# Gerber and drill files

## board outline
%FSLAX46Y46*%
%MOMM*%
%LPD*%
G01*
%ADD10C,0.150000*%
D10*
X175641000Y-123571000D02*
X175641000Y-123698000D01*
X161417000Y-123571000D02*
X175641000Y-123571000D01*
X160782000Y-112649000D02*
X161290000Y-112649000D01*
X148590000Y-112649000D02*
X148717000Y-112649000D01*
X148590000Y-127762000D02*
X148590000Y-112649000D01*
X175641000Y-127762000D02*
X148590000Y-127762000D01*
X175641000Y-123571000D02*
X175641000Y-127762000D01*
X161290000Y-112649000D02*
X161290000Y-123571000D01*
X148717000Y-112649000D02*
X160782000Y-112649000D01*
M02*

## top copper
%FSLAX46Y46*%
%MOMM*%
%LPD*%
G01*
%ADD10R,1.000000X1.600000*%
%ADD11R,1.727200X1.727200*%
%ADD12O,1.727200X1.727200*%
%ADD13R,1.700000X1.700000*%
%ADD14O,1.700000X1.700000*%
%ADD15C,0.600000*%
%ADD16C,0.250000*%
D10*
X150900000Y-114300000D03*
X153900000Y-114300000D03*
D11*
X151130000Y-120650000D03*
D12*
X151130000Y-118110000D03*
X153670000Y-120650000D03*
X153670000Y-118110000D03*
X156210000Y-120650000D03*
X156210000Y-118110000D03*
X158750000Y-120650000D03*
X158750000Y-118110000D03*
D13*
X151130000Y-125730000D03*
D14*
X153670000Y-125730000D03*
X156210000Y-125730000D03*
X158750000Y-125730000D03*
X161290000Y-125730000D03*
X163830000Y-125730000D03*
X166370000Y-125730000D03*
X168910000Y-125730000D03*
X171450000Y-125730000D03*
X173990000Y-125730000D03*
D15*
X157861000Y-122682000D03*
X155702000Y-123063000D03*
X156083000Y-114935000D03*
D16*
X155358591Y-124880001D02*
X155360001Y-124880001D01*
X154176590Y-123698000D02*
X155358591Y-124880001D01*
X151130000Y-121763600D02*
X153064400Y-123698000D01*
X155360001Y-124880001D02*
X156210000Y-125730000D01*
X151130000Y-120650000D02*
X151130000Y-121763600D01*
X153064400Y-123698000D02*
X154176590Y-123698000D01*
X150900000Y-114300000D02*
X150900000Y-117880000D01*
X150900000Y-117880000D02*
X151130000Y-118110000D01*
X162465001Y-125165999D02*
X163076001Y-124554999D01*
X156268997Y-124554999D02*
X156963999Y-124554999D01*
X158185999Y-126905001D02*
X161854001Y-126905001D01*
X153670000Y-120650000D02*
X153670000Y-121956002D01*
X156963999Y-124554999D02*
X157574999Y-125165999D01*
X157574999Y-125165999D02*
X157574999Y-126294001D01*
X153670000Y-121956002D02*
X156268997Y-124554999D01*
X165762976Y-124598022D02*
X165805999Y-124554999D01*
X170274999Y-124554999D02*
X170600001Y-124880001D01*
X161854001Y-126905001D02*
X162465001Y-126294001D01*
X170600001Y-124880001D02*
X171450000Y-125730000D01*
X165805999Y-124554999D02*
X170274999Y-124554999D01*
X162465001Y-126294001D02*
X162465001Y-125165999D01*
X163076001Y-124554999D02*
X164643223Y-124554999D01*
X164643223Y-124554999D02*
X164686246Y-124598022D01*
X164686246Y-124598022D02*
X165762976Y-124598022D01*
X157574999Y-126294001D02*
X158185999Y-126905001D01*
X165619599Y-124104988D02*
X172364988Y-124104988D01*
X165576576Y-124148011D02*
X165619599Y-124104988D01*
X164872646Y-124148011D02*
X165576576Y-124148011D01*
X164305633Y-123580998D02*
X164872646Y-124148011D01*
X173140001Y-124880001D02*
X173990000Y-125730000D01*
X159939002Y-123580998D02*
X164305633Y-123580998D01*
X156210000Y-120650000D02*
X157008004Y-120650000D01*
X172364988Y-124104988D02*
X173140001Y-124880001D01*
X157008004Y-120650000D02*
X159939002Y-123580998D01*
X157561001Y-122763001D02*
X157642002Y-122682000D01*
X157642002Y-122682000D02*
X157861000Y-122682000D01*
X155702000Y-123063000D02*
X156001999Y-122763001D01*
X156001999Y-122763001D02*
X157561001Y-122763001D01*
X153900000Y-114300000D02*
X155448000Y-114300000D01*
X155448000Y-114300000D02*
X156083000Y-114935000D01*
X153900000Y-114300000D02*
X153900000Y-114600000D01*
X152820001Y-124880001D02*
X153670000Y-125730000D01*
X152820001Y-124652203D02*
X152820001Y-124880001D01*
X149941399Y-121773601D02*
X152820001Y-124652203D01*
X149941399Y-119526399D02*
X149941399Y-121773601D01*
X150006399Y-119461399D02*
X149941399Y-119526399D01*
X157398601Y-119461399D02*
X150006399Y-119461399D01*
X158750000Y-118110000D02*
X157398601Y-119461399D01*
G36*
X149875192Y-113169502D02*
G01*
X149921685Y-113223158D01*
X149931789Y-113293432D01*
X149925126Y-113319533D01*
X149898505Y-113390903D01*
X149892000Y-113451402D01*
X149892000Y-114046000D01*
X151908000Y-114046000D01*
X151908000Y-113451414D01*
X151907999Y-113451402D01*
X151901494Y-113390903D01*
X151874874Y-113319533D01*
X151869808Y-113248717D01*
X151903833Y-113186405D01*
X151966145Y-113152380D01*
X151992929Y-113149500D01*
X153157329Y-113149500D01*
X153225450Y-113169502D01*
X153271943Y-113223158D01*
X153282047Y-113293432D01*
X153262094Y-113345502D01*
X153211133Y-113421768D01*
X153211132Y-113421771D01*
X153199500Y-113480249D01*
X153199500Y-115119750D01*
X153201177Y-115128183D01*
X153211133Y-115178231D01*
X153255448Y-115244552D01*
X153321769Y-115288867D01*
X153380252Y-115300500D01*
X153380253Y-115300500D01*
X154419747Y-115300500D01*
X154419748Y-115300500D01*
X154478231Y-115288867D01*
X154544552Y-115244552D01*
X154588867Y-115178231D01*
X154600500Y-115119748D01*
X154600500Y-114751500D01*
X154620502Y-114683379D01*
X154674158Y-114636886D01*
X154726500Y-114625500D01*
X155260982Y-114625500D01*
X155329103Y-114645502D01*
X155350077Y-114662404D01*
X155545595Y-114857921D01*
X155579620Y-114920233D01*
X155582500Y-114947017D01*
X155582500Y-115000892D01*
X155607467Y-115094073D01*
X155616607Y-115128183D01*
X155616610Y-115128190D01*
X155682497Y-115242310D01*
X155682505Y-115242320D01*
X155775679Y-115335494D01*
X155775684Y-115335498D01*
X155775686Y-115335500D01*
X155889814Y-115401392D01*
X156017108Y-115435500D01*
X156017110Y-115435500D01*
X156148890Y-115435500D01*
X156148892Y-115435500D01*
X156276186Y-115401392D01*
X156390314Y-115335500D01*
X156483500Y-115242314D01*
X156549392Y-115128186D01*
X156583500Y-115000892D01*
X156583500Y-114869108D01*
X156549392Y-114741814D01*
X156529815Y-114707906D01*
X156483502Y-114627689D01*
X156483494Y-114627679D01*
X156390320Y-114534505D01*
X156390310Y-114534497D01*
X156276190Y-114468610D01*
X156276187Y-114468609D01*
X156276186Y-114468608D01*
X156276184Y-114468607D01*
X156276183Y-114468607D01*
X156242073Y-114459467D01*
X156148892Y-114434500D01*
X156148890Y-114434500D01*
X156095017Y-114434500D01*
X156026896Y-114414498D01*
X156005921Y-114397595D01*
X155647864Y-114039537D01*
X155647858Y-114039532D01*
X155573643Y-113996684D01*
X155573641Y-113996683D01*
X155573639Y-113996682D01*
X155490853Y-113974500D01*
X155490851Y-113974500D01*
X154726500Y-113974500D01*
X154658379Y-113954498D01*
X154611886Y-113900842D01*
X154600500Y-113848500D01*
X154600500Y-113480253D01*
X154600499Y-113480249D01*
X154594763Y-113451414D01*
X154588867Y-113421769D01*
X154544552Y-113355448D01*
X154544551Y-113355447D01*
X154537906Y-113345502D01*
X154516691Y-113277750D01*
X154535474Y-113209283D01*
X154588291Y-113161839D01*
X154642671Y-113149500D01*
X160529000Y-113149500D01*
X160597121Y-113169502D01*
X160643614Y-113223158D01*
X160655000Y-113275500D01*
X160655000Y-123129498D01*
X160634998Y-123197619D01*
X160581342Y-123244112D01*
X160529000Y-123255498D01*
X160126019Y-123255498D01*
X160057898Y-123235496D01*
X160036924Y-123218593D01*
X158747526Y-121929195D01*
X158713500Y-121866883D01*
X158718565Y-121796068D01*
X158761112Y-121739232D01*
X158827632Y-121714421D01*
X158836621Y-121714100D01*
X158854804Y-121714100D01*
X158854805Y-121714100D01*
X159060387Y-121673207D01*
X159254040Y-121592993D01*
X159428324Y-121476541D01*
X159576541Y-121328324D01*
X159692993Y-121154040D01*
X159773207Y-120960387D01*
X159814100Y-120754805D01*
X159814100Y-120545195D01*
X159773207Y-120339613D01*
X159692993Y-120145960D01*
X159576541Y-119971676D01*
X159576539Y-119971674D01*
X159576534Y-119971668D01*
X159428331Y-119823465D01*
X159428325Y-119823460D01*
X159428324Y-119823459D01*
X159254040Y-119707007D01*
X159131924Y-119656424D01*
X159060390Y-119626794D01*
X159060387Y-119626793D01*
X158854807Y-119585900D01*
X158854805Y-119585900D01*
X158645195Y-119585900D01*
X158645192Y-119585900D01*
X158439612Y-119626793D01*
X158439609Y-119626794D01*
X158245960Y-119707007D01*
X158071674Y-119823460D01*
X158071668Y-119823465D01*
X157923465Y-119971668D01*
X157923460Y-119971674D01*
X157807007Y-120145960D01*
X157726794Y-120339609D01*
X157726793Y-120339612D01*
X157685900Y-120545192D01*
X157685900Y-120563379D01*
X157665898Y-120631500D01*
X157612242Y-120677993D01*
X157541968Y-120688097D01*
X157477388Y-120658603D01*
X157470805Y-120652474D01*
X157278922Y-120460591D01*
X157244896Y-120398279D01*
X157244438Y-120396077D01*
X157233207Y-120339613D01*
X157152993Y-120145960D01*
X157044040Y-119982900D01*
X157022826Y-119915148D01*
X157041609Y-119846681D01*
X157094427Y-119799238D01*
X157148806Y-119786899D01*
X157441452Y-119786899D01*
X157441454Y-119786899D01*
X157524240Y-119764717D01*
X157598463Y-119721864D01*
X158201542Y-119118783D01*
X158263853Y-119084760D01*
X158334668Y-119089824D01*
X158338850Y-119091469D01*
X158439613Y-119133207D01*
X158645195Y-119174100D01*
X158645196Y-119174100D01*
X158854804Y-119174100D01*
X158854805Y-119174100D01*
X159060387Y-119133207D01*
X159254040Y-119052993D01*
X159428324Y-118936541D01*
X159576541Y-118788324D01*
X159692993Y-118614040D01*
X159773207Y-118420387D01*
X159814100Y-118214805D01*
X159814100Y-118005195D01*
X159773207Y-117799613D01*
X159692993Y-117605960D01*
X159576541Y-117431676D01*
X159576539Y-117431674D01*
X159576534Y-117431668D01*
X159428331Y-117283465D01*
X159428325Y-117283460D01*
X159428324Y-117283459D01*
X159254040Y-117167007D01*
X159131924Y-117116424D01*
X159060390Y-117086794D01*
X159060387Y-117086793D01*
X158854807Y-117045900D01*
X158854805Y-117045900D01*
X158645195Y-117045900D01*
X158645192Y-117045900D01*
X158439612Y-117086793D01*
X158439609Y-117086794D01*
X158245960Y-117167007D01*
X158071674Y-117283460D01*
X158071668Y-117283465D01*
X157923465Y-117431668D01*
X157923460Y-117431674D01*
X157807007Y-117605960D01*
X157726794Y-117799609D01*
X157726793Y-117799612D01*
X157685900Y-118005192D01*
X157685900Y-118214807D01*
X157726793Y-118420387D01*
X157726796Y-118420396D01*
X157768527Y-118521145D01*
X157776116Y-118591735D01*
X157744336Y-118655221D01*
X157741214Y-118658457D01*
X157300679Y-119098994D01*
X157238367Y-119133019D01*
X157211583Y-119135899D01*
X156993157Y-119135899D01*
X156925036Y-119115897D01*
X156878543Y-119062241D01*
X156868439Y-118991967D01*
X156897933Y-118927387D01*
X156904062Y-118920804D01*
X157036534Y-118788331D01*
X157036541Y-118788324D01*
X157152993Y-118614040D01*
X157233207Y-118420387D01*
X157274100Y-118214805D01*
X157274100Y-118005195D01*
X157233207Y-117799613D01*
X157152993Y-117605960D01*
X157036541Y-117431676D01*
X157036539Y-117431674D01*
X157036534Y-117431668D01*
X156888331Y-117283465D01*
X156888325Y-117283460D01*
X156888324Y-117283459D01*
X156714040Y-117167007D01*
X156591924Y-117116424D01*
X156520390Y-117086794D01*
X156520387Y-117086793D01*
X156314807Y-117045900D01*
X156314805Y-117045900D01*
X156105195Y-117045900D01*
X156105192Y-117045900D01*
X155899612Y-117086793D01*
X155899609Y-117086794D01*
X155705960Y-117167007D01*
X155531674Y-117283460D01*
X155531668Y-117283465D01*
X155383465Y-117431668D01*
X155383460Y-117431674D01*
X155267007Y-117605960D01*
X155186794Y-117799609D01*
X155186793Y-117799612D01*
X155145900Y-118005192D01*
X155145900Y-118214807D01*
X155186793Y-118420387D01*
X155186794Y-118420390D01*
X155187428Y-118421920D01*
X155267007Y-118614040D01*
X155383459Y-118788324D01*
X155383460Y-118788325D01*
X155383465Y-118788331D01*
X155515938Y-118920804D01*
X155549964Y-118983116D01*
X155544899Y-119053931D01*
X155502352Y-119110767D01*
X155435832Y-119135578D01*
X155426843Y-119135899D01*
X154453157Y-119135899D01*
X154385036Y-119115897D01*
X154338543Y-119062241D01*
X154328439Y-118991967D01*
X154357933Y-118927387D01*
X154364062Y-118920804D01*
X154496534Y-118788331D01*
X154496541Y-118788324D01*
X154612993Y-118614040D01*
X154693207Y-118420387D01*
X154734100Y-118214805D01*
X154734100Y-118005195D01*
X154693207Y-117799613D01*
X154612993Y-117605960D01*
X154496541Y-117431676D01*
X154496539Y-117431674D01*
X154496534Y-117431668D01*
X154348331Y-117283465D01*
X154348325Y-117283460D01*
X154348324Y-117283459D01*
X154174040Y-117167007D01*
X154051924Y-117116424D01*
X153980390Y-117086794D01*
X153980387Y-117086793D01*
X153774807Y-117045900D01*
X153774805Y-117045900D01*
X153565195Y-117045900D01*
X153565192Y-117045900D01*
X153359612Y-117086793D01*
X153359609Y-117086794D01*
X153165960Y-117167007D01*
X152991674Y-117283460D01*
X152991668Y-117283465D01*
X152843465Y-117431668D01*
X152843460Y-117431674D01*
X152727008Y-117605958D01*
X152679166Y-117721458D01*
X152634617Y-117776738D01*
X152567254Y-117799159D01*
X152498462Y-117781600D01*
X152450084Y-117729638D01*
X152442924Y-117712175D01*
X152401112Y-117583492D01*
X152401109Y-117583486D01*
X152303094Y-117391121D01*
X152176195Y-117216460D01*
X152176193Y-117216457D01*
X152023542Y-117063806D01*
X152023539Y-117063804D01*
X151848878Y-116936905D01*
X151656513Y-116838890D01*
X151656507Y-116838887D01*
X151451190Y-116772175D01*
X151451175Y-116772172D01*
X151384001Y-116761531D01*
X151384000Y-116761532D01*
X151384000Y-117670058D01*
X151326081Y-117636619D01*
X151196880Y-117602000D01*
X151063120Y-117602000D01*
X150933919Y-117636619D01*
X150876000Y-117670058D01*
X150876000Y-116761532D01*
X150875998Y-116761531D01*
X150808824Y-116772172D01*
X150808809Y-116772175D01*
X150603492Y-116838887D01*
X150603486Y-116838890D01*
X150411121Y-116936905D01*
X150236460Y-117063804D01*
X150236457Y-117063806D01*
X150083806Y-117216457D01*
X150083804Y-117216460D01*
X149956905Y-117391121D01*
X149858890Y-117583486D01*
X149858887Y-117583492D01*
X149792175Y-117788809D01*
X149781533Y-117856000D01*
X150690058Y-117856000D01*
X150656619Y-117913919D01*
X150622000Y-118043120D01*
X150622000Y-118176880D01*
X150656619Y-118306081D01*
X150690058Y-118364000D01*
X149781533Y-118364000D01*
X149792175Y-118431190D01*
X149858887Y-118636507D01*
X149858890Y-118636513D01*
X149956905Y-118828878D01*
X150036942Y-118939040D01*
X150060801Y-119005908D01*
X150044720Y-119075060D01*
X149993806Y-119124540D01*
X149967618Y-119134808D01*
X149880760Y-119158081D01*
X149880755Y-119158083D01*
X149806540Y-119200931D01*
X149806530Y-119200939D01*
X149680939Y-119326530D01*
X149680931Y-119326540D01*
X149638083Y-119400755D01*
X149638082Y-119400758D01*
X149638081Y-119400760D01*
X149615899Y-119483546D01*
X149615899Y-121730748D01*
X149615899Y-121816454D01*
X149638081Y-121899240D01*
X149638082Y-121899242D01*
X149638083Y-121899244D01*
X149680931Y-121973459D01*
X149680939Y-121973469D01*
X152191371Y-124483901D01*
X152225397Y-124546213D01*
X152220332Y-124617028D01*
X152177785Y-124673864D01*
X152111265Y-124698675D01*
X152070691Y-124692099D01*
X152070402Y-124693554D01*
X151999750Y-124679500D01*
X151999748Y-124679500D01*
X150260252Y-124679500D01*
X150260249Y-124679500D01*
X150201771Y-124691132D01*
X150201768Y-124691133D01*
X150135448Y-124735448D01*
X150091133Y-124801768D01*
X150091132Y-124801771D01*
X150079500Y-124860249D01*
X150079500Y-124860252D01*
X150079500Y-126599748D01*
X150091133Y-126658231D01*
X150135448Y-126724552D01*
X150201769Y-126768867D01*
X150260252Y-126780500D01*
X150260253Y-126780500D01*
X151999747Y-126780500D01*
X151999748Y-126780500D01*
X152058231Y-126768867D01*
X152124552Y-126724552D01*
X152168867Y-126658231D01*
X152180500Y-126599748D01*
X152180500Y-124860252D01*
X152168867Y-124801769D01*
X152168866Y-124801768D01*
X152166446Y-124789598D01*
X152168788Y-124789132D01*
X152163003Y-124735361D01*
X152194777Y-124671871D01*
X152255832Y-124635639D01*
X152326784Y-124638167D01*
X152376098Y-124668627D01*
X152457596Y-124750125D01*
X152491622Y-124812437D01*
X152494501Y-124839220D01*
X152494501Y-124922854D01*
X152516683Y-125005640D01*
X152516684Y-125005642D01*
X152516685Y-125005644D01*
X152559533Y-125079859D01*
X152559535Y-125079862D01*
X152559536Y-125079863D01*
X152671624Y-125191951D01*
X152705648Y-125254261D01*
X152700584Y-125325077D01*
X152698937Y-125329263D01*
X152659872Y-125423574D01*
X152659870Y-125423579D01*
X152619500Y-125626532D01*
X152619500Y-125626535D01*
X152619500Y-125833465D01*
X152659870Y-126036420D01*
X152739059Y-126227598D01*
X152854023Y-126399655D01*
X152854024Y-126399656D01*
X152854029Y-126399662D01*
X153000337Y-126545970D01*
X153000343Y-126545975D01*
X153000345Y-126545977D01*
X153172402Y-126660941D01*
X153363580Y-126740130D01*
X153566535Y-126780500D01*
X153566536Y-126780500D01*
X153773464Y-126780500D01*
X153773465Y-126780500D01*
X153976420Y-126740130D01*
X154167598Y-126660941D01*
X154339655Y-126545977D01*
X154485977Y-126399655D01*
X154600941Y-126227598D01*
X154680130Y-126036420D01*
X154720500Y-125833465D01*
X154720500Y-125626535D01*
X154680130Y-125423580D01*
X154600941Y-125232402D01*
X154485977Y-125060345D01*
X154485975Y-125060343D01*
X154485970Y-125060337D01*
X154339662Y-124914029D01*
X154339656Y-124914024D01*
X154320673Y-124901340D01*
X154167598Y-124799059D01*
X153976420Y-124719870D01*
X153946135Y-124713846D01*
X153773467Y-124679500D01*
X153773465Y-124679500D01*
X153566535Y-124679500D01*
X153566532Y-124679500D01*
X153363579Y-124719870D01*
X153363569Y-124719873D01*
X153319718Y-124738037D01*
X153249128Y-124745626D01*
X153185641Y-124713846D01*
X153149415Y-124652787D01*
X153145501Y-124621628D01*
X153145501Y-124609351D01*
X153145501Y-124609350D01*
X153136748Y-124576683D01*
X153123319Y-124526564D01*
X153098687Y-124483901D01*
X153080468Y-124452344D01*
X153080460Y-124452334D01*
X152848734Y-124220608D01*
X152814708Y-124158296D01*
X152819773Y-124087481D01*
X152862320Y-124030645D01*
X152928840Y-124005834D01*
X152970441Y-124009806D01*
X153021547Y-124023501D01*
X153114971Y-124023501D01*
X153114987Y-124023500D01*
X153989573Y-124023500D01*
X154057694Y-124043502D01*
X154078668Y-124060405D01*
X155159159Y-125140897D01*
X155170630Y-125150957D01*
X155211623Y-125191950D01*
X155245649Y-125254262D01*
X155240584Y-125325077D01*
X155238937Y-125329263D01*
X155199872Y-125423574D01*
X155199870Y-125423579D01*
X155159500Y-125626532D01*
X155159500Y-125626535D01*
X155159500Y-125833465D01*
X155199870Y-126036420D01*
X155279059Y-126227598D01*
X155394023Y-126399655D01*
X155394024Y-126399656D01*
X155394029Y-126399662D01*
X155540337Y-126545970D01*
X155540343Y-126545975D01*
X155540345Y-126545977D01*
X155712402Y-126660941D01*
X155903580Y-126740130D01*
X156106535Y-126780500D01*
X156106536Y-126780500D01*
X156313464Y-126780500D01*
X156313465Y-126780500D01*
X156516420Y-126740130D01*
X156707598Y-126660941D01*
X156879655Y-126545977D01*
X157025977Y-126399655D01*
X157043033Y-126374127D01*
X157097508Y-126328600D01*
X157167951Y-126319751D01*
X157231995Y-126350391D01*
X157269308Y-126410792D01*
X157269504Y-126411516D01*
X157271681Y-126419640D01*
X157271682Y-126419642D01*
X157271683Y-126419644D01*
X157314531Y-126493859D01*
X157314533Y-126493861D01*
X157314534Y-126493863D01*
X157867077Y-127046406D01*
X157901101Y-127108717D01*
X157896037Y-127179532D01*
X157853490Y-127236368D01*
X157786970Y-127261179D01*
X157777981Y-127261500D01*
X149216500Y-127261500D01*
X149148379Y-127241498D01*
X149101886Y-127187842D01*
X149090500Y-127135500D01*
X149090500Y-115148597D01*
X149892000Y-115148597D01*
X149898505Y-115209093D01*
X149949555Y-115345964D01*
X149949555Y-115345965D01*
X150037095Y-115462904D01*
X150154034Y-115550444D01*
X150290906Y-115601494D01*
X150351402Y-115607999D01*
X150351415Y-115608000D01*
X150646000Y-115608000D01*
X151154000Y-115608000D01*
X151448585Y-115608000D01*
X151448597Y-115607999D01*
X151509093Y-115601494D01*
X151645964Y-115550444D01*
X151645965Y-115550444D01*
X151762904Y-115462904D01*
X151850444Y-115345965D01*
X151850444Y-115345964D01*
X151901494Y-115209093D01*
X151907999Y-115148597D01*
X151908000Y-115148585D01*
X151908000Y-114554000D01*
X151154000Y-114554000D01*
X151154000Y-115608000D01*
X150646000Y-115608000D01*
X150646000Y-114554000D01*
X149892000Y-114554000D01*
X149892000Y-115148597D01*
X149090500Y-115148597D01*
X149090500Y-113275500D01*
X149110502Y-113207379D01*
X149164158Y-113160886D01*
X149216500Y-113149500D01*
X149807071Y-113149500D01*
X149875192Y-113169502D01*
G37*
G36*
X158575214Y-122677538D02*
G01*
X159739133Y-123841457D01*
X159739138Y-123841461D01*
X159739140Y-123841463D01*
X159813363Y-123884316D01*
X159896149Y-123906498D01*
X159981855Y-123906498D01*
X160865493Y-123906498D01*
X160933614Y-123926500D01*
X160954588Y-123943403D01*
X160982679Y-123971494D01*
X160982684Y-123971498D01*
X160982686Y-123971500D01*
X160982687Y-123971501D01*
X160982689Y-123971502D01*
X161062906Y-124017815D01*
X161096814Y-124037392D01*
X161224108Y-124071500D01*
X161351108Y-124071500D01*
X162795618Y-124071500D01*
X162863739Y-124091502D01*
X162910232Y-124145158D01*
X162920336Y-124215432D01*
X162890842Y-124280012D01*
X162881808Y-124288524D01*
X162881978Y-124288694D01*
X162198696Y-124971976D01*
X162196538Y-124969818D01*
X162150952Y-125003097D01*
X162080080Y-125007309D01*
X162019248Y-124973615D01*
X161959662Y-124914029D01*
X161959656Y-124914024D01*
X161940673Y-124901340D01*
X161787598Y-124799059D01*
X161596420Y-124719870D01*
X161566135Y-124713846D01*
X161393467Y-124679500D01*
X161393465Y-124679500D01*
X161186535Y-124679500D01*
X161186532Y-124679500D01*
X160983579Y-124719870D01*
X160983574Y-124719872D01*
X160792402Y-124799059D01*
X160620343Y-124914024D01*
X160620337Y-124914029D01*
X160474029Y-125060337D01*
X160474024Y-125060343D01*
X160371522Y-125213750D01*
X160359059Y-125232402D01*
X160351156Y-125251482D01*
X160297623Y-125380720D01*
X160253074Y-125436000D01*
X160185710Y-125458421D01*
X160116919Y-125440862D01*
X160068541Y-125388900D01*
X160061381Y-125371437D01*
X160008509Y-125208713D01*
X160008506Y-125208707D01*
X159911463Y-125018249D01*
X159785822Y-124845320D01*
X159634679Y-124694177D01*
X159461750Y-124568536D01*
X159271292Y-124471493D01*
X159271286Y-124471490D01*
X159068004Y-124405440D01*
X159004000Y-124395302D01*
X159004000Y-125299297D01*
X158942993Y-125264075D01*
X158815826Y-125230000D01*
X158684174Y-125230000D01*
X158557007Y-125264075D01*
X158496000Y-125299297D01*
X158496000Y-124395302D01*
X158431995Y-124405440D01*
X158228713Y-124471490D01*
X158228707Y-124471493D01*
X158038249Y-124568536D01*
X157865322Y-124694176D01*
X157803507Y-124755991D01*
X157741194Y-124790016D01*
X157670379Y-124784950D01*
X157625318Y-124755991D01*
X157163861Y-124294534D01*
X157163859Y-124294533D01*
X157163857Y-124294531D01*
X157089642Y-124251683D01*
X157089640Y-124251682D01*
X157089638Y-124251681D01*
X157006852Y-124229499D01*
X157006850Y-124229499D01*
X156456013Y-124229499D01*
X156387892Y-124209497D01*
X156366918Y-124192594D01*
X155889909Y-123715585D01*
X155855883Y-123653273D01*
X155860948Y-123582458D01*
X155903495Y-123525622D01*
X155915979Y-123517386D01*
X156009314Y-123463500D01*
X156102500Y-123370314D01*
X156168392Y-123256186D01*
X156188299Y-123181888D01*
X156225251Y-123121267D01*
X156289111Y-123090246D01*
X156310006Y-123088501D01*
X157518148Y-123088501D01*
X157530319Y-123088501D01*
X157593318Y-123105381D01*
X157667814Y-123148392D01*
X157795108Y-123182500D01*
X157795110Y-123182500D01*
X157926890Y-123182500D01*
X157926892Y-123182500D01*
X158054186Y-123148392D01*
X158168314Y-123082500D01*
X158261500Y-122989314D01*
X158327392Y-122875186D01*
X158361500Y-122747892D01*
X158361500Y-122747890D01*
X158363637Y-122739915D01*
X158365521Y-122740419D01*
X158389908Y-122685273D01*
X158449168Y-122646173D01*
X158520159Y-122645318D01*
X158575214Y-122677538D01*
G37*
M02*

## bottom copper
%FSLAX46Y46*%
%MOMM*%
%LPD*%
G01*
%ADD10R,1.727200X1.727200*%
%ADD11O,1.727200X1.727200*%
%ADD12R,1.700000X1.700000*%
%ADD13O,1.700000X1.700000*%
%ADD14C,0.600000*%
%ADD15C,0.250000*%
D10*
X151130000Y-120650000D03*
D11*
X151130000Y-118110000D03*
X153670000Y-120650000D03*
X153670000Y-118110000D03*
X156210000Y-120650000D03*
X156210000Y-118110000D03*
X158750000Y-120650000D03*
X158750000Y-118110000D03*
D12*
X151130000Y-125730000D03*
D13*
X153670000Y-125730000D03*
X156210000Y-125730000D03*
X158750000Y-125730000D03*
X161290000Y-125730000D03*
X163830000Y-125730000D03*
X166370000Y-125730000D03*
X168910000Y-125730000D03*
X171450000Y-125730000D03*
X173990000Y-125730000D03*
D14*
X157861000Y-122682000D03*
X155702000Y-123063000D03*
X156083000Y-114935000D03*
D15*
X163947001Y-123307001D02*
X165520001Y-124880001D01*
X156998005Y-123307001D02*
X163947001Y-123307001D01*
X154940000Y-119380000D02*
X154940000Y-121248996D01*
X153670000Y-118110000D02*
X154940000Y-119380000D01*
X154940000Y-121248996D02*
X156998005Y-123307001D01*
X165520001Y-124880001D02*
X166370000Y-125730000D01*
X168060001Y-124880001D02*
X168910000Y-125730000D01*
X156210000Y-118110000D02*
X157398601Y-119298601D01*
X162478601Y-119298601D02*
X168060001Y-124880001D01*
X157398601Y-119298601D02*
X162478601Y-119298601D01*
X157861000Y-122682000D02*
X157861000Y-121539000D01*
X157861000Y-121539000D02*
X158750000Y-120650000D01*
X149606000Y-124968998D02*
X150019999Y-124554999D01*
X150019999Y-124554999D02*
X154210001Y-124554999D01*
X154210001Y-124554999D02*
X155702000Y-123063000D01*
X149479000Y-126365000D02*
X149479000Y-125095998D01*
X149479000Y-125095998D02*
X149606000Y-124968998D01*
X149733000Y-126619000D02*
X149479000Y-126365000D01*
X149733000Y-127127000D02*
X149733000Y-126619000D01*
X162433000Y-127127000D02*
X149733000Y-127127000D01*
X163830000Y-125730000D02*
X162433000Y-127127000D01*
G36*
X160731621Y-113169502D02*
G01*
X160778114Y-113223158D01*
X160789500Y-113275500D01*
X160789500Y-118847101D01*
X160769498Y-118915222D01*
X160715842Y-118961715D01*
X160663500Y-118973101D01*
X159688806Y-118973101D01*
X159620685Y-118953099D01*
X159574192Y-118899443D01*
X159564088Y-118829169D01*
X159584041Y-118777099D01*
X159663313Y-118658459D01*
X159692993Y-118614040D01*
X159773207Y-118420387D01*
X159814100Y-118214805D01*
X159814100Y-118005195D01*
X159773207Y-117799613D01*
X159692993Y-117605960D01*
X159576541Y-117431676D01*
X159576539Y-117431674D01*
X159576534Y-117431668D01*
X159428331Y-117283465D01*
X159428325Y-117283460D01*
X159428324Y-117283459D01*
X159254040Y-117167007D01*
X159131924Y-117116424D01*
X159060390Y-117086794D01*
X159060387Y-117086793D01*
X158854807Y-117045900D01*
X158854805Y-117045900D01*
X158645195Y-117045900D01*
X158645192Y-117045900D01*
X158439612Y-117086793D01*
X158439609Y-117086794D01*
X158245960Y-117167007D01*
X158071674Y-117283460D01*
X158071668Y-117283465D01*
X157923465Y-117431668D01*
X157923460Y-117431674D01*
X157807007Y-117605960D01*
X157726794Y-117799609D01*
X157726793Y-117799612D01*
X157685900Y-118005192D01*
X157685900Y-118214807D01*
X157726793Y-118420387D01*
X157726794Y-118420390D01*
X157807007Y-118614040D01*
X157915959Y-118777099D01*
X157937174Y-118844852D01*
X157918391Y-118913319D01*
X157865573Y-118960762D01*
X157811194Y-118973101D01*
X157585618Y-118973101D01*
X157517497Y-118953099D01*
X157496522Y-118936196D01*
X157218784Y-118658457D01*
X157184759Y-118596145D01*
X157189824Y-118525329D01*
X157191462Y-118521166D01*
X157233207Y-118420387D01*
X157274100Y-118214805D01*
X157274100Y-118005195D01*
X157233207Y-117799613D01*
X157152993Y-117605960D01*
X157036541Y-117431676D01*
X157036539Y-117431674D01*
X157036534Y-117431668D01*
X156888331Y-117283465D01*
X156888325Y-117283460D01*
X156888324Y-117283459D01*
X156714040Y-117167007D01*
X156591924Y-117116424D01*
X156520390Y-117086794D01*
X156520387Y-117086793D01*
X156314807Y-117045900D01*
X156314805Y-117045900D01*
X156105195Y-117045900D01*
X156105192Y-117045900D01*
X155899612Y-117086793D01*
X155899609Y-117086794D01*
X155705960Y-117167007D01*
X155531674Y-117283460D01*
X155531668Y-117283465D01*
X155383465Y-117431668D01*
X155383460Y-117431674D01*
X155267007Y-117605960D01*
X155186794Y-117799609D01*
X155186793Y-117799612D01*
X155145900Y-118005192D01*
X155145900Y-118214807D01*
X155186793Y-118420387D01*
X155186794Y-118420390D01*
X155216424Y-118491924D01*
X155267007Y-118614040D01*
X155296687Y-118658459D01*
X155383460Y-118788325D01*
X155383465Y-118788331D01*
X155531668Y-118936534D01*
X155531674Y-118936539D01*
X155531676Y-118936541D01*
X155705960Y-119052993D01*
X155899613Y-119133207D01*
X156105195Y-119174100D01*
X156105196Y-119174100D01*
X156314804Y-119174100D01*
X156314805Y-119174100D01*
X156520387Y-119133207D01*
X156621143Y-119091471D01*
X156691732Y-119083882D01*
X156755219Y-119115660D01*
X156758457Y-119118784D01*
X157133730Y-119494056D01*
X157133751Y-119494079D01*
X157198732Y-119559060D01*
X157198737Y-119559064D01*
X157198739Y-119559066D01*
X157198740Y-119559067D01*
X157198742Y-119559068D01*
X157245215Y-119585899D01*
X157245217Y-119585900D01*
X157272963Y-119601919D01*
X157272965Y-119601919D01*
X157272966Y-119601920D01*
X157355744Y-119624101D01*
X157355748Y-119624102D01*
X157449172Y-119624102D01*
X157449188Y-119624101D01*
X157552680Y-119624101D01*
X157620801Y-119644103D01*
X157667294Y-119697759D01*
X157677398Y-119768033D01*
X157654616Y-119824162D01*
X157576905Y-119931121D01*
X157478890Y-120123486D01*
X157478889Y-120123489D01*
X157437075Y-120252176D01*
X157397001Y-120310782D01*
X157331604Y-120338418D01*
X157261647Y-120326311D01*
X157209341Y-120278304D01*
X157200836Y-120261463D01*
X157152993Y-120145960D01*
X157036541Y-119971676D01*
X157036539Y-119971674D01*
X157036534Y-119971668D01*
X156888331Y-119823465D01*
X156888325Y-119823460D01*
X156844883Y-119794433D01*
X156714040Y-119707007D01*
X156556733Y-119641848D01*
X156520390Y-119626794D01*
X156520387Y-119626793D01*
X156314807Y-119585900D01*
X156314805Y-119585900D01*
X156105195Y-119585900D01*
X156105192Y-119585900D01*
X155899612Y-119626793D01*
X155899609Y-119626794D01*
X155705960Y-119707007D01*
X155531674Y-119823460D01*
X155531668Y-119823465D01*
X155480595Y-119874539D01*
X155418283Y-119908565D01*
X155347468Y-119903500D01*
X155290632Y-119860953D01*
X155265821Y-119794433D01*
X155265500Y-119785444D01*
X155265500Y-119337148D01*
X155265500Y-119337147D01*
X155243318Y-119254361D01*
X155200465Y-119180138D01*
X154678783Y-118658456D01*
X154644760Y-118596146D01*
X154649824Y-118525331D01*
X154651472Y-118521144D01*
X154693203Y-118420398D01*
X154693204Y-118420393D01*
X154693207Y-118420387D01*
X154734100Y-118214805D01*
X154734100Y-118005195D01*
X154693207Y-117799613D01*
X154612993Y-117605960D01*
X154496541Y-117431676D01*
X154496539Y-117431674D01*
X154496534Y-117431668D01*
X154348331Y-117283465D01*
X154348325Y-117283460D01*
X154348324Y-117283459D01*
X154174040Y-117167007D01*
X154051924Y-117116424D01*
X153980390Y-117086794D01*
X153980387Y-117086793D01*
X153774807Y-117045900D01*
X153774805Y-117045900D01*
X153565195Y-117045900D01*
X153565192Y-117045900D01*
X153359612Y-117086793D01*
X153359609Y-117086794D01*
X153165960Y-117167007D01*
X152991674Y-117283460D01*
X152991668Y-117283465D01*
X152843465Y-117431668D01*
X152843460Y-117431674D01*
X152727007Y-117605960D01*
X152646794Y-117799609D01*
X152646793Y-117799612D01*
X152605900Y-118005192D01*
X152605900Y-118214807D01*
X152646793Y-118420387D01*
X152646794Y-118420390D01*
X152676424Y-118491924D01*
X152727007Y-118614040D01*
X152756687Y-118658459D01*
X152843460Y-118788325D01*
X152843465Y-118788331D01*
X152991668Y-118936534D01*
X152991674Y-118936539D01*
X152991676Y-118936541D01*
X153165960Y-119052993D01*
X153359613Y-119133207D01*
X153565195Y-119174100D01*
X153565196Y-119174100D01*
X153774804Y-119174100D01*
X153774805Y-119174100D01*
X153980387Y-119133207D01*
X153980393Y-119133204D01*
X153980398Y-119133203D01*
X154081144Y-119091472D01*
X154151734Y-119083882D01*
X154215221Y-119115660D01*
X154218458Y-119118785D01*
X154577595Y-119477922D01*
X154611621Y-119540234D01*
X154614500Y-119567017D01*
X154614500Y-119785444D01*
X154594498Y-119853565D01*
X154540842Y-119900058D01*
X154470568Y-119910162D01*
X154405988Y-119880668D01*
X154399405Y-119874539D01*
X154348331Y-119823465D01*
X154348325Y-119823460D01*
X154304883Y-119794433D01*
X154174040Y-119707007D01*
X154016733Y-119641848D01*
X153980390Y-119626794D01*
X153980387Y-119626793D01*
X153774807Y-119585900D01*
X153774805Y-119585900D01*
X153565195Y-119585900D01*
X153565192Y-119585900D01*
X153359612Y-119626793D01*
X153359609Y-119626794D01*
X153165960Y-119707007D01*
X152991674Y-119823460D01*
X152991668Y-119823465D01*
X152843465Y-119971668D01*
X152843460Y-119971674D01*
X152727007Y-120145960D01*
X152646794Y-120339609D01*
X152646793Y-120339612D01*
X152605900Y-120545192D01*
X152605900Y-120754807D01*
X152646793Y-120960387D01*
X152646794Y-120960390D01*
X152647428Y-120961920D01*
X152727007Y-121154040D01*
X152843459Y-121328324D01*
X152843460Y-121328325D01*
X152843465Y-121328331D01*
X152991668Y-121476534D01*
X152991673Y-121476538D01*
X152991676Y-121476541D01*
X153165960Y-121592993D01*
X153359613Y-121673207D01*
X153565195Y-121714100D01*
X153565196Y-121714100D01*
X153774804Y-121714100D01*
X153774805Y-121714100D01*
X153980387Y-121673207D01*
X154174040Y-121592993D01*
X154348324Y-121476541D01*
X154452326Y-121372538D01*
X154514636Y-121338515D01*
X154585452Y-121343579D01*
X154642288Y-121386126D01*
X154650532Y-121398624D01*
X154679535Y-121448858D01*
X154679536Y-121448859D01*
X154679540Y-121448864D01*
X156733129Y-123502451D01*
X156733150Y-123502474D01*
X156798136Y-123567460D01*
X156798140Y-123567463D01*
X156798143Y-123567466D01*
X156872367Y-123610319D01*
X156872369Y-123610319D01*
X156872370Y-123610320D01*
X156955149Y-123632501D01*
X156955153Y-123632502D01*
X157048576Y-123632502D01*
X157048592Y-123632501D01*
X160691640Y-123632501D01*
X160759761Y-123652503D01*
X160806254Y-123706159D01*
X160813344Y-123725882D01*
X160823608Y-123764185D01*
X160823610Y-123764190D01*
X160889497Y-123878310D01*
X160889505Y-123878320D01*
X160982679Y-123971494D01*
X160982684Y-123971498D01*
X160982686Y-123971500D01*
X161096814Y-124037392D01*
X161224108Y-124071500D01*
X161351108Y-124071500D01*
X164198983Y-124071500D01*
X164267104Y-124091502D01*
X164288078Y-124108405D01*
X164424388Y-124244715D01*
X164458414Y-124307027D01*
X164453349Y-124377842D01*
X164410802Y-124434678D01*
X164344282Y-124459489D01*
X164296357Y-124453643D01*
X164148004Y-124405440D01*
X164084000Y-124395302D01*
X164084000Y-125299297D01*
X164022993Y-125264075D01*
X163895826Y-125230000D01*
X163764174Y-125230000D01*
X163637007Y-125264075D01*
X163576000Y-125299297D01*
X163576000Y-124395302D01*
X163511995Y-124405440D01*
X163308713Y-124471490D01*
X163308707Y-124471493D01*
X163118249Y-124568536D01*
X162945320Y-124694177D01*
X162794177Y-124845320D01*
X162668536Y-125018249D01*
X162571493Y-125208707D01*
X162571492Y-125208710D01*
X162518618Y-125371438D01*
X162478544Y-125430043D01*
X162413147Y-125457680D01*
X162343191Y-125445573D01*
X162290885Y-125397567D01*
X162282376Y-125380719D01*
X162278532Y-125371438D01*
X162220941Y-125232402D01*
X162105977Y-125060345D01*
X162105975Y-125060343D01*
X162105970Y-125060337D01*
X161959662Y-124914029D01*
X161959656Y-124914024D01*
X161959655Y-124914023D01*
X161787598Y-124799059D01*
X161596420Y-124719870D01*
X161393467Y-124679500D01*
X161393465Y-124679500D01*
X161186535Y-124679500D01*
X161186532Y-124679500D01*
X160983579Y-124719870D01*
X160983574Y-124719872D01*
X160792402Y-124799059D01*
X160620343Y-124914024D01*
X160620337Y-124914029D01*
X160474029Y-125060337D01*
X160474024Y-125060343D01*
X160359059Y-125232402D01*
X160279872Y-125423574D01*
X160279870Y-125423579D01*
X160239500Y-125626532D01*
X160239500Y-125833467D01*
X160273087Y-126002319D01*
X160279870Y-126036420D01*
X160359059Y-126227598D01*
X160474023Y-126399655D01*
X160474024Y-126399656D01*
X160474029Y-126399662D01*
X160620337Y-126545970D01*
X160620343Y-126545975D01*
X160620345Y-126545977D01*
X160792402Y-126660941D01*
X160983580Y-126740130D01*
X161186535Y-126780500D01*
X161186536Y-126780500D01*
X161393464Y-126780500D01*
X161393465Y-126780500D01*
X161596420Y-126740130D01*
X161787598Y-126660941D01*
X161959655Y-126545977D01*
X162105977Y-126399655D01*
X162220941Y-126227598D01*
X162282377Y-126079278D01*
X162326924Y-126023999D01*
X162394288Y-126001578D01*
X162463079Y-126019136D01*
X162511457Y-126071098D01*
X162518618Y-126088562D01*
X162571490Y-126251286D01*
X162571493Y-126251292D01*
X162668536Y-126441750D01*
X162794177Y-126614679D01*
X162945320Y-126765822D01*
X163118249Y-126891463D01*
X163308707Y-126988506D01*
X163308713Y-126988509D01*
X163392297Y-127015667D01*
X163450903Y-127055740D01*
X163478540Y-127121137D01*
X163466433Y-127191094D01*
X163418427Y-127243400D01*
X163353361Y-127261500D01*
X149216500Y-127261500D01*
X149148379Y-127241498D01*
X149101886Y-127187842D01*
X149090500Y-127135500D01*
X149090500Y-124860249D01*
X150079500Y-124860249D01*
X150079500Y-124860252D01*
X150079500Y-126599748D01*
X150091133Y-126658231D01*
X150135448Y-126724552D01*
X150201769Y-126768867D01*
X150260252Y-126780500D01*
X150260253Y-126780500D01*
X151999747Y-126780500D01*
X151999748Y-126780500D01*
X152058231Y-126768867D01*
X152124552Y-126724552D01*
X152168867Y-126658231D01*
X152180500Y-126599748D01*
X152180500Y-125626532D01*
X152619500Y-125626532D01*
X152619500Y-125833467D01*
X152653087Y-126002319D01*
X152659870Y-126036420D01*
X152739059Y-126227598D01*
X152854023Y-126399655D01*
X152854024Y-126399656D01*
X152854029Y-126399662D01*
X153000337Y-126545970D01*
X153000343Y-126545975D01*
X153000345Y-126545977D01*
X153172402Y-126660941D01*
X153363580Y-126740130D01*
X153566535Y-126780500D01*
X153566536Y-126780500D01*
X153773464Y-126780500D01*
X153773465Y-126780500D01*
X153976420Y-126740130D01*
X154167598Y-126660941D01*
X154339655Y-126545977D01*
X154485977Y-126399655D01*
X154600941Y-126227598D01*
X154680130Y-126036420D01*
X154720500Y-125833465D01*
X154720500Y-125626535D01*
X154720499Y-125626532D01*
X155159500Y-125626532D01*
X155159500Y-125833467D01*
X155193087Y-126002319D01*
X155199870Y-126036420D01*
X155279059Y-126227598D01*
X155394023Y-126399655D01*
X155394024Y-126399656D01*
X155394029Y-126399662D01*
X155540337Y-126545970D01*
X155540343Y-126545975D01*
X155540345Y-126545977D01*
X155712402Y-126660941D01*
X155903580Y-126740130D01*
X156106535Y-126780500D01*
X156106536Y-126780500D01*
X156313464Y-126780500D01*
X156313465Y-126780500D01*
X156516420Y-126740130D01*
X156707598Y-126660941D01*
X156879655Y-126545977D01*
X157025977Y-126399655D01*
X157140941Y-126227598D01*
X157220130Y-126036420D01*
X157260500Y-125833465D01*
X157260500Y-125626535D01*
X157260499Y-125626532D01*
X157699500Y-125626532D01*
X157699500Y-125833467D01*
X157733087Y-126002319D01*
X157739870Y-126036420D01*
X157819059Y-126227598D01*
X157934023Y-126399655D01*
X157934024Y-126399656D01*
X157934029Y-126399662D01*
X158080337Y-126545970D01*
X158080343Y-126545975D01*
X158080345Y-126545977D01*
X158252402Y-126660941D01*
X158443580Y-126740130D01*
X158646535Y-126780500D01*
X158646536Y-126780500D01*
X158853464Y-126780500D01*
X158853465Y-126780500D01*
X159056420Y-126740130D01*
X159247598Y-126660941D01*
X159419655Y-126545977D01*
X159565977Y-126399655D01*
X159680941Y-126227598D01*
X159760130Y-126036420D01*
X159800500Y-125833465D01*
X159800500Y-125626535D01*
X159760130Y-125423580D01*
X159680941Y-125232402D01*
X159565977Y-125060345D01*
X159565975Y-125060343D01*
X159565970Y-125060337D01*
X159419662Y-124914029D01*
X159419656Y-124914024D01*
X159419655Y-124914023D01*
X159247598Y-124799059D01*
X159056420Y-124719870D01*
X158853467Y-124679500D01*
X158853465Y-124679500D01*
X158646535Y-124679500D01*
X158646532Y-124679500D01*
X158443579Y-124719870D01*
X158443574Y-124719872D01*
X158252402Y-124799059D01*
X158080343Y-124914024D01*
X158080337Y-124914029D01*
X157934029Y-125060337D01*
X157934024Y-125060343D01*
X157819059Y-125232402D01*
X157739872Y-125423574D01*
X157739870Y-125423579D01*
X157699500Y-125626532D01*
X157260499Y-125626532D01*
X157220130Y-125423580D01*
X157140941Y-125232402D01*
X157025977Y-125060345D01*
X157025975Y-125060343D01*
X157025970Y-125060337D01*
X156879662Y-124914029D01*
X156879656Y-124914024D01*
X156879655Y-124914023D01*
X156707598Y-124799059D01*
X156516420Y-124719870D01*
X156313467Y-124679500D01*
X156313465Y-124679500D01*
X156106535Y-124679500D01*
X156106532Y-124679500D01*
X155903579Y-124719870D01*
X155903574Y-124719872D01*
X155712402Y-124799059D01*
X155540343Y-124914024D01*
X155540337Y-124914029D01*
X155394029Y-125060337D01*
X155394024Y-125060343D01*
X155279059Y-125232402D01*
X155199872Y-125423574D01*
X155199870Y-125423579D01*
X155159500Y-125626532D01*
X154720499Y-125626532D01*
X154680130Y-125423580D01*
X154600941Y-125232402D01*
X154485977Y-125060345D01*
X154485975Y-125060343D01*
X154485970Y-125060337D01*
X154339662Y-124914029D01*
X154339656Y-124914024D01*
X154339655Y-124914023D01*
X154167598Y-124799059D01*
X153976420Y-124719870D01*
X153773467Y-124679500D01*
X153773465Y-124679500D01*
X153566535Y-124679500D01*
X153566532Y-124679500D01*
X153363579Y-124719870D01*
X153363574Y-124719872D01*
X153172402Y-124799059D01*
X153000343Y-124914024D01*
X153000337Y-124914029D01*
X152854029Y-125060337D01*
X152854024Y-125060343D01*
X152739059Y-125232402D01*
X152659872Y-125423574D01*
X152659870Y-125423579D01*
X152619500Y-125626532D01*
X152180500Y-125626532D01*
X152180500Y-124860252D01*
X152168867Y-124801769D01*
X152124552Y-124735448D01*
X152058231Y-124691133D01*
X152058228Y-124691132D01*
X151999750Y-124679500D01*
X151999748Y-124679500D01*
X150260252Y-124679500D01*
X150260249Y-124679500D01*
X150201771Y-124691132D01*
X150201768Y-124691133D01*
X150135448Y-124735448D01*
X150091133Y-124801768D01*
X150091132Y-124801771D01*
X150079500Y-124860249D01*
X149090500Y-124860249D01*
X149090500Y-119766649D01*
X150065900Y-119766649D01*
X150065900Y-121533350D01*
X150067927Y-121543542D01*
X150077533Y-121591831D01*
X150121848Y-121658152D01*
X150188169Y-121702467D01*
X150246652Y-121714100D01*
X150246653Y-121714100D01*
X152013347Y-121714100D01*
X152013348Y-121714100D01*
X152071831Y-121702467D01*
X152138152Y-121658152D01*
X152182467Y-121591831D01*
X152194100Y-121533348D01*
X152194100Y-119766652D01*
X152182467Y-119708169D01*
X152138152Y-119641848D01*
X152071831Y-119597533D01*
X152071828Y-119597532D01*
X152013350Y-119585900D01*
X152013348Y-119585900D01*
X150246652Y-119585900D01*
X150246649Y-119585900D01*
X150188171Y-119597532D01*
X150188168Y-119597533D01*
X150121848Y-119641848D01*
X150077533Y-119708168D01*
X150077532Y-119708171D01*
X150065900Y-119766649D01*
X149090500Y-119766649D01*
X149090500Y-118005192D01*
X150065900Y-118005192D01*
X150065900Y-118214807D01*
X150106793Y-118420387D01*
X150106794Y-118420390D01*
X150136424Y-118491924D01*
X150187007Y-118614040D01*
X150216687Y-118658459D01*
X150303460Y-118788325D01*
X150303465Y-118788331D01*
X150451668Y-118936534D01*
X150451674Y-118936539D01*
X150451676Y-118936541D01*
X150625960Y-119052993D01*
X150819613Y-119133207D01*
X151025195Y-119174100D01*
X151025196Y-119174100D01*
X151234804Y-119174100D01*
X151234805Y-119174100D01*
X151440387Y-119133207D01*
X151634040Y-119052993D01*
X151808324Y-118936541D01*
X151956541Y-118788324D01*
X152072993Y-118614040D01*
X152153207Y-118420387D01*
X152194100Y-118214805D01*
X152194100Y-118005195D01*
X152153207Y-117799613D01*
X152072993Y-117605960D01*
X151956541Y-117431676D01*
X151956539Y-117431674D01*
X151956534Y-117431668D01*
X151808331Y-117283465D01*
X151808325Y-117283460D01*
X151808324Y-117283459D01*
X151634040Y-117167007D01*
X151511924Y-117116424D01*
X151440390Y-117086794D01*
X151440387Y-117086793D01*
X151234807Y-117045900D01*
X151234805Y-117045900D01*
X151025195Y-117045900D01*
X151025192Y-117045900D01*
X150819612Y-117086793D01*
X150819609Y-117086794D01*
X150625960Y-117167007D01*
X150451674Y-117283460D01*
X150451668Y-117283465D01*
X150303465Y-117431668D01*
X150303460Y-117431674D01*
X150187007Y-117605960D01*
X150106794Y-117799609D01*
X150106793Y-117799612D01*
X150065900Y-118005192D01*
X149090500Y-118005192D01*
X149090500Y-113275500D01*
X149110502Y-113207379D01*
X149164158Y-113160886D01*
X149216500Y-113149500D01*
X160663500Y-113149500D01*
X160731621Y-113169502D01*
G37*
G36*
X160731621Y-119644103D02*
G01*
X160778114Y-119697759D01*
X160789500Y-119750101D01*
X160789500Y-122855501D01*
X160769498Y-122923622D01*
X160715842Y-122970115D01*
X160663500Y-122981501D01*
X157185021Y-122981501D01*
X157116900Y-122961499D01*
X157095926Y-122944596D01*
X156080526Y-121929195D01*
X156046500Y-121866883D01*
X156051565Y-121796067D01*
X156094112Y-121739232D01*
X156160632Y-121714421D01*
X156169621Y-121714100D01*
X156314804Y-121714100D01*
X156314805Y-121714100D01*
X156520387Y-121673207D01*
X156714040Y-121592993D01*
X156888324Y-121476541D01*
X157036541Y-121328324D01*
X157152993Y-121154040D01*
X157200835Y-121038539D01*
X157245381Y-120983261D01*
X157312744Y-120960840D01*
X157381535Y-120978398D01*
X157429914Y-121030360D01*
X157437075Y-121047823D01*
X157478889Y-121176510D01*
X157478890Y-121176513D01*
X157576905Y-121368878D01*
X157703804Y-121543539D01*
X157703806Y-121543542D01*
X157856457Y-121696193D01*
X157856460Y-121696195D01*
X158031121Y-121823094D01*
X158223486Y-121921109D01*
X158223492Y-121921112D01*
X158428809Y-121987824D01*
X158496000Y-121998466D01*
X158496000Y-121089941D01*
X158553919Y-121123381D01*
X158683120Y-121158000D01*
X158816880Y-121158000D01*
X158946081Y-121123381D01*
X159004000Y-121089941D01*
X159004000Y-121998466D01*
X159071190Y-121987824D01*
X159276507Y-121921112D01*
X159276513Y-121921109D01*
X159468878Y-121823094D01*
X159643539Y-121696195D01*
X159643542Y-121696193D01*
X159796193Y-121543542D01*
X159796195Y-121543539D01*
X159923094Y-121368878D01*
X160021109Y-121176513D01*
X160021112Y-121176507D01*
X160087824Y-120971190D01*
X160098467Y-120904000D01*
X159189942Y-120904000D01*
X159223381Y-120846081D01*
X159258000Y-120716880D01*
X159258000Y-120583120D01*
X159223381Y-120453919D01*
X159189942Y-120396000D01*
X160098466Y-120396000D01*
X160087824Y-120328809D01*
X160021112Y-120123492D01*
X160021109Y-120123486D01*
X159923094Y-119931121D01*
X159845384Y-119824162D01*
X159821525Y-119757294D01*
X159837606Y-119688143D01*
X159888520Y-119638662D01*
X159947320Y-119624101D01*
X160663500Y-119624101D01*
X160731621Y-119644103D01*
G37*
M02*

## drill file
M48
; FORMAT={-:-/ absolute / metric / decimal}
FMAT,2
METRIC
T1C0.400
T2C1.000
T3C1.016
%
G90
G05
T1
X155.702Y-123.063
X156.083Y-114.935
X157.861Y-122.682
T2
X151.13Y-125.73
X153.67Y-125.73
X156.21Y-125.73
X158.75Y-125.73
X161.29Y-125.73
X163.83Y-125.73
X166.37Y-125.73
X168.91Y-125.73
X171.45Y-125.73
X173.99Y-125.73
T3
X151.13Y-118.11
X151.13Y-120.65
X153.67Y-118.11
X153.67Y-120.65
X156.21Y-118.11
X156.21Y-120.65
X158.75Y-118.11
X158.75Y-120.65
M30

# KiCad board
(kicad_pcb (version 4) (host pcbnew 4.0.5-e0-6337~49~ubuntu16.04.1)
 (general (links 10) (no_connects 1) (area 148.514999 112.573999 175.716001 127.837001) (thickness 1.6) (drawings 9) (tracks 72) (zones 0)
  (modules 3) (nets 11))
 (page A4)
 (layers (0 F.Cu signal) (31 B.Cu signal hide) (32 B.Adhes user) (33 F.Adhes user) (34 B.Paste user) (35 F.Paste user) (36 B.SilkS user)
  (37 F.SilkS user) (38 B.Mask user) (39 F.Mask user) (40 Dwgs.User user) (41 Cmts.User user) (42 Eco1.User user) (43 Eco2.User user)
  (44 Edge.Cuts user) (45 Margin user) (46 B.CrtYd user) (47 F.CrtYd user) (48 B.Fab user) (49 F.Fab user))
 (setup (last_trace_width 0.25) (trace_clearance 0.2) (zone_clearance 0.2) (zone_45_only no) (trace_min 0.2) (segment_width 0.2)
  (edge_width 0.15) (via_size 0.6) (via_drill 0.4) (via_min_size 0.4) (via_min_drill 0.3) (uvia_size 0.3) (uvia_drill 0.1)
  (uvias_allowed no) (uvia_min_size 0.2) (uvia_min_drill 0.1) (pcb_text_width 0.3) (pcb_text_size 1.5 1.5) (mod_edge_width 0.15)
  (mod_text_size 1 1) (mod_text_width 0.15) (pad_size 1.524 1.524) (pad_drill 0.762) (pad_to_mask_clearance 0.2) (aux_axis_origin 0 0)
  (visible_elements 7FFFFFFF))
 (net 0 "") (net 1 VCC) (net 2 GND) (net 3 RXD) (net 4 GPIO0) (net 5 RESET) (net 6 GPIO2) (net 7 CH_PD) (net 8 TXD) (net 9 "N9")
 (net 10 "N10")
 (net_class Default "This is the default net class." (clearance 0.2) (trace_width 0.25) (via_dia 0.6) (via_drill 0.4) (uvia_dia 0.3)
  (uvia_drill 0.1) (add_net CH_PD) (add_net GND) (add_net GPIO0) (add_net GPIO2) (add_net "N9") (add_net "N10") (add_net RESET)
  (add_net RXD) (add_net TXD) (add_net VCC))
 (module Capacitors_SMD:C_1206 (layer F.Cu) (at 152.4 114.3)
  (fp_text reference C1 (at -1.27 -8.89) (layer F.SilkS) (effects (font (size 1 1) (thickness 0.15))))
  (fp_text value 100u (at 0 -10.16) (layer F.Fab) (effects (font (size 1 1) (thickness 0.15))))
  (pad 1 smd rect (at -1.5 0) (size 1 1.6) (layers F.Cu F.Paste F.Mask) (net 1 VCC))
  (pad 2 smd rect (at 1.5 0) (size 1 1.6) (layers F.Cu F.Paste F.Mask) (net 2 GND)))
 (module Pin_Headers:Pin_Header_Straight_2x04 (layer F.Cu) (at 151.13 120.65 90)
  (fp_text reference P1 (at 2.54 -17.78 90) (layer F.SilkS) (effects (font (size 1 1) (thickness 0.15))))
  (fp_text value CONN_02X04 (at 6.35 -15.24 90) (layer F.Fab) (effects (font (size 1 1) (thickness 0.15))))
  (pad 1 thru_hole rect (at 0 0 90) (size 1.7272 1.7272) (drill 1.016) (layers *.Cu *.Mask) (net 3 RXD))
  (pad 2 thru_hole oval (at 2.54 0 90) (size 1.7272 1.7272) (drill 1.016) (layers *.Cu *.Mask) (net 1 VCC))
  (pad 3 thru_hole oval (at 0 2.54 90) (size 1.7272 1.7272) (drill 1.016) (layers *.Cu *.Mask) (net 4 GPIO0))
  (pad 4 thru_hole oval (at 2.54 2.54 90) (size 1.7272 1.7272) (drill 1.016) (layers *.Cu *.Mask) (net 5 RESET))
  (pad 5 thru_hole oval (at 0 5.08 90) (size 1.7272 1.7272) (drill 1.016) (layers *.Cu *.Mask) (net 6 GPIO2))
  (pad 6 thru_hole oval (at 2.54 5.08 90) (size 1.7272 1.7272) (drill 1.016) (layers *.Cu *.Mask) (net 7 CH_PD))
  (pad 7 thru_hole oval (at 0 7.62 90) (size 1.7272 1.7272) (drill 1.016) (layers *.Cu *.Mask) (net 2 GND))
  (pad 8 thru_hole oval (at 2.54 7.62 90) (size 1.7272 1.7272) (drill 1.016) (layers *.Cu *.Mask) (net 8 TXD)))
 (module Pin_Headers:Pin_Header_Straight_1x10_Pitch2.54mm (layer F.Cu) (at 151.13 125.73 90)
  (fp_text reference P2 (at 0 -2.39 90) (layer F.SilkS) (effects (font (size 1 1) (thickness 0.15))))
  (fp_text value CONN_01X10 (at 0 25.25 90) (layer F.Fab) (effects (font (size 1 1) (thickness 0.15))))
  (pad 1 thru_hole rect (at 0 0 90) (size 1.7 1.7) (drill 1) (layers *.Cu *.Mask) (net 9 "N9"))
  (pad 2 thru_hole oval (at 0 2.54 90) (size 1.7 1.7) (drill 1) (layers *.Cu *.Mask) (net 8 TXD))
  (pad 3 thru_hole oval (at 0 5.08 90) (size 1.7 1.7) (drill 1) (layers *.Cu *.Mask) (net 3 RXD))
  (pad 4 thru_hole oval (at 0 7.62 90) (size 1.7 1.7) (drill 1) (layers *.Cu *.Mask) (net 1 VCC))
  (pad 5 thru_hole oval (at 0 10.16 90) (size 1.7 1.7) (drill 1) (layers *.Cu *.Mask) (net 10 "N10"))
  (pad 6 thru_hole oval (at 0 12.7 90) (size 1.7 1.7) (drill 1) (layers *.Cu *.Mask) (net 2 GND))
  (pad 7 thru_hole oval (at 0 15.24 90) (size 1.7 1.7) (drill 1) (layers *.Cu *.Mask) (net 5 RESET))
  (pad 8 thru_hole oval (at 0 17.78 90) (size 1.7 1.7) (drill 1) (layers *.Cu *.Mask) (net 7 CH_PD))
  (pad 9 thru_hole oval (at 0 20.32 90) (size 1.7 1.7) (drill 1) (layers *.Cu *.Mask) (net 4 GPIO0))
  (pad 10 thru_hole oval (at 0 22.86 90) (size 1.7 1.7) (drill 1) (layers *.Cu *.Mask) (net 6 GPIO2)))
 (gr_line (start 175.641 123.571) (end 175.641 123.698) (angle 90) (layer Edge.Cuts) (width 0.15))
 (gr_line (start 161.417 123.571) (end 175.641 123.571) (angle 90) (layer Edge.Cuts) (width 0.15))
 (gr_line (start 160.782 112.649) (end 161.29 112.649) (angle 90) (layer Edge.Cuts) (width 0.15))
 (gr_line (start 148.59 112.649) (end 148.717 112.649) (angle 90) (layer Edge.Cuts) (width 0.15))
 (gr_line (start 148.59 127.762) (end 148.59 112.649) (angle 90) (layer Edge.Cuts) (width 0.15))
 (gr_line (start 175.641 127.762) (end 148.59 127.762) (angle 90) (layer Edge.Cuts) (width 0.15))
 (gr_line (start 175.641 123.571) (end 175.641 127.762) (angle 90) (layer Edge.Cuts) (width 0.15))
 (gr_line (start 161.29 112.649) (end 161.29 123.571) (angle 90) (layer Edge.Cuts) (width 0.15))
 (gr_line (start 148.717 112.649) (end 160.782 112.649) (angle 90) (layer Edge.Cuts) (width 0.15))
 (segment (start 155.358591 124.880001) (end 155.360001 124.880001) (width 0.25) (layer F.Cu) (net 3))
 (segment (start 154.17659 123.698) (end 155.358591 124.880001) (width 0.25) (layer F.Cu) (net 3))
 (segment (start 151.13 121.7636) (end 153.0644 123.698) (width 0.25) (layer F.Cu) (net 3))
 (segment (start 155.360001 124.880001) (end 156.21 125.73) (width 0.25) (layer F.Cu) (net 3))
 (segment (start 151.13 120.65) (end 151.13 121.7636) (width 0.25) (layer F.Cu) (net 3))
 (segment (start 153.0644 123.698) (end 154.17659 123.698) (width 0.25) (layer F.Cu) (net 3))
 (segment (start 150.9 114.3) (end 150.9 117.88) (width 0.25) (layer F.Cu) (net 1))
 (segment (start 150.9 117.88) (end 151.13 118.11) (width 0.25) (layer F.Cu) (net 1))
 (segment (start 162.465001 125.165999) (end 163.076001 124.554999) (width 0.25) (layer F.Cu) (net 4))
 (segment (start 156.268997 124.554999) (end 156.963999 124.554999) (width 0.25) (layer F.Cu) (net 4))
 (segment (start 158.185999 126.905001) (end 161.854001 126.905001) (width 0.25) (layer F.Cu) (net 4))
 (segment (start 153.67 120.65) (end 153.67 121.956002) (width 0.25) (layer F.Cu) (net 4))
 (segment (start 156.963999 124.554999) (end 157.574999 125.165999) (width 0.25) (layer F.Cu) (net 4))
 (segment (start 157.574999 125.165999) (end 157.574999 126.294001) (width 0.25) (layer F.Cu) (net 4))
 (segment (start 153.67 121.956002) (end 156.268997 124.554999) (width 0.25) (layer F.Cu) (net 4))
 (segment (start 165.762976 124.598022) (end 165.805999 124.554999) (width 0.25) (layer F.Cu) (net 4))
 (segment (start 170.274999 124.554999) (end 170.600001 124.880001) (width 0.25) (layer F.Cu) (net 4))
 (segment (start 161.854001 126.905001) (end 162.465001 126.294001) (width 0.25) (layer F.Cu) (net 4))
 (segment (start 170.600001 124.880001) (end 171.45 125.73) (width 0.25) (layer F.Cu) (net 4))
 (segment (start 165.805999 124.554999) (end 170.274999 124.554999) (width 0.25) (layer F.Cu) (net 4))
 (segment (start 162.465001 126.294001) (end 162.465001 125.165999) (width 0.25) (layer F.Cu) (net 4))
 (segment (start 163.076001 124.554999) (end 164.643223 124.554999) (width 0.25) (layer F.Cu) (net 4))
 (segment (start 164.643223 124.554999) (end 164.686246 124.598022) (width 0.25) (layer F.Cu) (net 4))
 (segment (start 164.686246 124.598022) (end 165.762976 124.598022) (width 0.25) (layer F.Cu) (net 4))
 (segment (start 157.574999 126.294001) (end 158.185999 126.905001) (width 0.25) (layer F.Cu) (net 4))
 (segment (start 163.947001 123.307001) (end 165.520001 124.880001) (width 0.25) (layer B.Cu) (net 5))
 (segment (start 156.998005 123.307001) (end 163.947001 123.307001) (width 0.25) (layer B.Cu) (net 5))
 (segment (start 154.94 119.38) (end 154.94 121.248996) (width 0.25) (layer B.Cu) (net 5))
 (segment (start 153.67 118.11) (end 154.94 119.38) (width 0.25) (layer B.Cu) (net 5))
 (segment (start 154.94 121.248996) (end 156.998005 123.307001) (width 0.25) (layer B.Cu) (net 5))
 (segment (start 165.520001 124.880001) (end 166.37 125.73) (width 0.25) (layer B.Cu) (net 5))
 (segment (start 165.619599 124.104988) (end 172.364988 124.104988) (width 0.25) (layer F.Cu) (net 6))
 (segment (start 165.576576 124.148011) (end 165.619599 124.104988) (width 0.25) (layer F.Cu) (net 6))
 (segment (start 164.872646 124.148011) (end 165.576576 124.148011) (width 0.25) (layer F.Cu) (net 6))
 (segment (start 164.305633 123.580998) (end 164.872646 124.148011) (width 0.25) (layer F.Cu) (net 6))
 (segment (start 173.140001 124.880001) (end 173.99 125.73) (width 0.25) (layer F.Cu) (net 6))
 (segment (start 159.939002 123.580998) (end 164.305633 123.580998) (width 0.25) (layer F.Cu) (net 6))
 (segment (start 156.21 120.65) (end 157.008004 120.65) (width 0.25) (layer F.Cu) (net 6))
 (segment (start 172.364988 124.104988) (end 173.140001 124.880001) (width 0.25) (layer F.Cu) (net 6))
 (segment (start 157.008004 120.65) (end 159.939002 123.580998) (width 0.25) (layer F.Cu) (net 6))
 (segment (start 168.060001 124.880001) (end 168.91 125.73) (width 0.25) (layer B.Cu) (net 7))
 (segment (start 156.21 118.11) (end 157.398601 119.298601) (width 0.25) (layer B.Cu) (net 7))
 (segment (start 162.478601 119.298601) (end 168.060001 124.880001) (width 0.25) (layer B.Cu) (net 7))
 (segment (start 157.398601 119.298601) (end 162.478601 119.298601) (width 0.25) (layer B.Cu) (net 7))
 (segment (start 157.861 122.682) (end 157.861 121.539) (width 0.25) (layer B.Cu) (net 2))
 (segment (start 157.861 121.539) (end 158.75 120.65) (width 0.25) (layer B.Cu) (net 2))
 (via (at 157.861 122.682) (size 0.6) (drill 0.4) (layers F.Cu B.Cu) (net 2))
 (segment (start 157.561001 122.763001) (end 157.642002 122.682) (width 0.25) (layer F.Cu) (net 2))
 (segment (start 157.642002 122.682) (end 157.861 122.682) (width 0.25) (layer F.Cu) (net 2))
 (segment (start 155.702 123.063) (end 156.001999 122.763001) (width 0.25) (layer F.Cu) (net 2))
 (segment (start 156.001999 122.763001) (end 157.561001 122.763001) (width 0.25) (layer F.Cu) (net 2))
 (segment (start 149.606 124.968998) (end 150.019999 124.554999) (width 0.25) (layer B.Cu) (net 2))
 (segment (start 150.019999 124.554999) (end 154.210001 124.554999) (width 0.25) (layer B.Cu) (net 2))
 (segment (start 154.210001 124.554999) (end 155.702 123.063) (width 0.25) (layer B.Cu) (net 2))
 (via (at 155.702 123.063) (size 0.6) (drill 0.4) (layers F.Cu B.Cu) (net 2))
 (segment (start 149.479 126.365) (end 149.479 125.095998) (width 0.25) (layer B.Cu) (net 2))
 (segment (start 149.479 125.095998) (end 149.606 124.968998) (width 0.25) (layer B.Cu) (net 2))
 (segment (start 149.733 126.619) (end 149.479 126.365) (width 0.25) (layer B.Cu) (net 2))
 (segment (start 149.733 127.127) (end 149.733 126.619) (width 0.25) (layer B.Cu) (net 2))
 (segment (start 162.433 127.127) (end 149.733 127.127) (width 0.25) (layer B.Cu) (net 2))
 (segment (start 163.83 125.73) (end 162.433 127.127) (width 0.25) (layer B.Cu) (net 2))
 (segment (start 153.9 114.3) (end 155.448 114.3) (width 0.25) (layer F.Cu) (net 2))
 (via (at 156.083 114.935) (size 0.6) (drill 0.4) (layers F.Cu B.Cu) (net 2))
 (segment (start 155.448 114.3) (end 156.083 114.935) (width 0.25) (layer F.Cu) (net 2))
 (segment (start 153.9 114.3) (end 153.9 114.6) (width 0.25) (layer F.Cu) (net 2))
 (segment (start 152.820001 124.880001) (end 153.67 125.73) (width 0.25) (layer F.Cu) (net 8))
 (segment (start 152.820001 124.652203) (end 152.820001 124.880001) (width 0.25) (layer F.Cu) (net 8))
 (segment (start 149.941399 121.773601) (end 152.820001 124.652203) (width 0.25) (layer F.Cu) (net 8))
 (segment (start 149.941399 119.526399) (end 149.941399 121.773601) (width 0.25) (layer F.Cu) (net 8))
 (segment (start 150.006399 119.461399) (end 149.941399 119.526399) (width 0.25) (layer F.Cu) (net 8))
 (segment (start 157.398601 119.461399) (end 150.006399 119.461399) (width 0.25) (layer F.Cu) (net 8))
 (segment (start 158.75 118.11) (end 157.398601 119.461399) (width 0.25) (layer F.Cu) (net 8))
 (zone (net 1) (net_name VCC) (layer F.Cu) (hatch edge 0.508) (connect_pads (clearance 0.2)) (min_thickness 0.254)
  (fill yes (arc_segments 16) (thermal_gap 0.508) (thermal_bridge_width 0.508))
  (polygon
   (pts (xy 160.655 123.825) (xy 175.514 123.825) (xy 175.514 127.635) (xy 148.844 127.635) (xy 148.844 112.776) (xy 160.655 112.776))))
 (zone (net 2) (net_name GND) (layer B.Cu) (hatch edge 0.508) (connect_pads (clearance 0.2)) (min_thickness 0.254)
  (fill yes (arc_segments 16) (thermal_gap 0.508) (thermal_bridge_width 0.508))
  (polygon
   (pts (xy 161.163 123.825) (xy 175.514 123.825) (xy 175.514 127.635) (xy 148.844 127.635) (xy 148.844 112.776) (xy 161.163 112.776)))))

